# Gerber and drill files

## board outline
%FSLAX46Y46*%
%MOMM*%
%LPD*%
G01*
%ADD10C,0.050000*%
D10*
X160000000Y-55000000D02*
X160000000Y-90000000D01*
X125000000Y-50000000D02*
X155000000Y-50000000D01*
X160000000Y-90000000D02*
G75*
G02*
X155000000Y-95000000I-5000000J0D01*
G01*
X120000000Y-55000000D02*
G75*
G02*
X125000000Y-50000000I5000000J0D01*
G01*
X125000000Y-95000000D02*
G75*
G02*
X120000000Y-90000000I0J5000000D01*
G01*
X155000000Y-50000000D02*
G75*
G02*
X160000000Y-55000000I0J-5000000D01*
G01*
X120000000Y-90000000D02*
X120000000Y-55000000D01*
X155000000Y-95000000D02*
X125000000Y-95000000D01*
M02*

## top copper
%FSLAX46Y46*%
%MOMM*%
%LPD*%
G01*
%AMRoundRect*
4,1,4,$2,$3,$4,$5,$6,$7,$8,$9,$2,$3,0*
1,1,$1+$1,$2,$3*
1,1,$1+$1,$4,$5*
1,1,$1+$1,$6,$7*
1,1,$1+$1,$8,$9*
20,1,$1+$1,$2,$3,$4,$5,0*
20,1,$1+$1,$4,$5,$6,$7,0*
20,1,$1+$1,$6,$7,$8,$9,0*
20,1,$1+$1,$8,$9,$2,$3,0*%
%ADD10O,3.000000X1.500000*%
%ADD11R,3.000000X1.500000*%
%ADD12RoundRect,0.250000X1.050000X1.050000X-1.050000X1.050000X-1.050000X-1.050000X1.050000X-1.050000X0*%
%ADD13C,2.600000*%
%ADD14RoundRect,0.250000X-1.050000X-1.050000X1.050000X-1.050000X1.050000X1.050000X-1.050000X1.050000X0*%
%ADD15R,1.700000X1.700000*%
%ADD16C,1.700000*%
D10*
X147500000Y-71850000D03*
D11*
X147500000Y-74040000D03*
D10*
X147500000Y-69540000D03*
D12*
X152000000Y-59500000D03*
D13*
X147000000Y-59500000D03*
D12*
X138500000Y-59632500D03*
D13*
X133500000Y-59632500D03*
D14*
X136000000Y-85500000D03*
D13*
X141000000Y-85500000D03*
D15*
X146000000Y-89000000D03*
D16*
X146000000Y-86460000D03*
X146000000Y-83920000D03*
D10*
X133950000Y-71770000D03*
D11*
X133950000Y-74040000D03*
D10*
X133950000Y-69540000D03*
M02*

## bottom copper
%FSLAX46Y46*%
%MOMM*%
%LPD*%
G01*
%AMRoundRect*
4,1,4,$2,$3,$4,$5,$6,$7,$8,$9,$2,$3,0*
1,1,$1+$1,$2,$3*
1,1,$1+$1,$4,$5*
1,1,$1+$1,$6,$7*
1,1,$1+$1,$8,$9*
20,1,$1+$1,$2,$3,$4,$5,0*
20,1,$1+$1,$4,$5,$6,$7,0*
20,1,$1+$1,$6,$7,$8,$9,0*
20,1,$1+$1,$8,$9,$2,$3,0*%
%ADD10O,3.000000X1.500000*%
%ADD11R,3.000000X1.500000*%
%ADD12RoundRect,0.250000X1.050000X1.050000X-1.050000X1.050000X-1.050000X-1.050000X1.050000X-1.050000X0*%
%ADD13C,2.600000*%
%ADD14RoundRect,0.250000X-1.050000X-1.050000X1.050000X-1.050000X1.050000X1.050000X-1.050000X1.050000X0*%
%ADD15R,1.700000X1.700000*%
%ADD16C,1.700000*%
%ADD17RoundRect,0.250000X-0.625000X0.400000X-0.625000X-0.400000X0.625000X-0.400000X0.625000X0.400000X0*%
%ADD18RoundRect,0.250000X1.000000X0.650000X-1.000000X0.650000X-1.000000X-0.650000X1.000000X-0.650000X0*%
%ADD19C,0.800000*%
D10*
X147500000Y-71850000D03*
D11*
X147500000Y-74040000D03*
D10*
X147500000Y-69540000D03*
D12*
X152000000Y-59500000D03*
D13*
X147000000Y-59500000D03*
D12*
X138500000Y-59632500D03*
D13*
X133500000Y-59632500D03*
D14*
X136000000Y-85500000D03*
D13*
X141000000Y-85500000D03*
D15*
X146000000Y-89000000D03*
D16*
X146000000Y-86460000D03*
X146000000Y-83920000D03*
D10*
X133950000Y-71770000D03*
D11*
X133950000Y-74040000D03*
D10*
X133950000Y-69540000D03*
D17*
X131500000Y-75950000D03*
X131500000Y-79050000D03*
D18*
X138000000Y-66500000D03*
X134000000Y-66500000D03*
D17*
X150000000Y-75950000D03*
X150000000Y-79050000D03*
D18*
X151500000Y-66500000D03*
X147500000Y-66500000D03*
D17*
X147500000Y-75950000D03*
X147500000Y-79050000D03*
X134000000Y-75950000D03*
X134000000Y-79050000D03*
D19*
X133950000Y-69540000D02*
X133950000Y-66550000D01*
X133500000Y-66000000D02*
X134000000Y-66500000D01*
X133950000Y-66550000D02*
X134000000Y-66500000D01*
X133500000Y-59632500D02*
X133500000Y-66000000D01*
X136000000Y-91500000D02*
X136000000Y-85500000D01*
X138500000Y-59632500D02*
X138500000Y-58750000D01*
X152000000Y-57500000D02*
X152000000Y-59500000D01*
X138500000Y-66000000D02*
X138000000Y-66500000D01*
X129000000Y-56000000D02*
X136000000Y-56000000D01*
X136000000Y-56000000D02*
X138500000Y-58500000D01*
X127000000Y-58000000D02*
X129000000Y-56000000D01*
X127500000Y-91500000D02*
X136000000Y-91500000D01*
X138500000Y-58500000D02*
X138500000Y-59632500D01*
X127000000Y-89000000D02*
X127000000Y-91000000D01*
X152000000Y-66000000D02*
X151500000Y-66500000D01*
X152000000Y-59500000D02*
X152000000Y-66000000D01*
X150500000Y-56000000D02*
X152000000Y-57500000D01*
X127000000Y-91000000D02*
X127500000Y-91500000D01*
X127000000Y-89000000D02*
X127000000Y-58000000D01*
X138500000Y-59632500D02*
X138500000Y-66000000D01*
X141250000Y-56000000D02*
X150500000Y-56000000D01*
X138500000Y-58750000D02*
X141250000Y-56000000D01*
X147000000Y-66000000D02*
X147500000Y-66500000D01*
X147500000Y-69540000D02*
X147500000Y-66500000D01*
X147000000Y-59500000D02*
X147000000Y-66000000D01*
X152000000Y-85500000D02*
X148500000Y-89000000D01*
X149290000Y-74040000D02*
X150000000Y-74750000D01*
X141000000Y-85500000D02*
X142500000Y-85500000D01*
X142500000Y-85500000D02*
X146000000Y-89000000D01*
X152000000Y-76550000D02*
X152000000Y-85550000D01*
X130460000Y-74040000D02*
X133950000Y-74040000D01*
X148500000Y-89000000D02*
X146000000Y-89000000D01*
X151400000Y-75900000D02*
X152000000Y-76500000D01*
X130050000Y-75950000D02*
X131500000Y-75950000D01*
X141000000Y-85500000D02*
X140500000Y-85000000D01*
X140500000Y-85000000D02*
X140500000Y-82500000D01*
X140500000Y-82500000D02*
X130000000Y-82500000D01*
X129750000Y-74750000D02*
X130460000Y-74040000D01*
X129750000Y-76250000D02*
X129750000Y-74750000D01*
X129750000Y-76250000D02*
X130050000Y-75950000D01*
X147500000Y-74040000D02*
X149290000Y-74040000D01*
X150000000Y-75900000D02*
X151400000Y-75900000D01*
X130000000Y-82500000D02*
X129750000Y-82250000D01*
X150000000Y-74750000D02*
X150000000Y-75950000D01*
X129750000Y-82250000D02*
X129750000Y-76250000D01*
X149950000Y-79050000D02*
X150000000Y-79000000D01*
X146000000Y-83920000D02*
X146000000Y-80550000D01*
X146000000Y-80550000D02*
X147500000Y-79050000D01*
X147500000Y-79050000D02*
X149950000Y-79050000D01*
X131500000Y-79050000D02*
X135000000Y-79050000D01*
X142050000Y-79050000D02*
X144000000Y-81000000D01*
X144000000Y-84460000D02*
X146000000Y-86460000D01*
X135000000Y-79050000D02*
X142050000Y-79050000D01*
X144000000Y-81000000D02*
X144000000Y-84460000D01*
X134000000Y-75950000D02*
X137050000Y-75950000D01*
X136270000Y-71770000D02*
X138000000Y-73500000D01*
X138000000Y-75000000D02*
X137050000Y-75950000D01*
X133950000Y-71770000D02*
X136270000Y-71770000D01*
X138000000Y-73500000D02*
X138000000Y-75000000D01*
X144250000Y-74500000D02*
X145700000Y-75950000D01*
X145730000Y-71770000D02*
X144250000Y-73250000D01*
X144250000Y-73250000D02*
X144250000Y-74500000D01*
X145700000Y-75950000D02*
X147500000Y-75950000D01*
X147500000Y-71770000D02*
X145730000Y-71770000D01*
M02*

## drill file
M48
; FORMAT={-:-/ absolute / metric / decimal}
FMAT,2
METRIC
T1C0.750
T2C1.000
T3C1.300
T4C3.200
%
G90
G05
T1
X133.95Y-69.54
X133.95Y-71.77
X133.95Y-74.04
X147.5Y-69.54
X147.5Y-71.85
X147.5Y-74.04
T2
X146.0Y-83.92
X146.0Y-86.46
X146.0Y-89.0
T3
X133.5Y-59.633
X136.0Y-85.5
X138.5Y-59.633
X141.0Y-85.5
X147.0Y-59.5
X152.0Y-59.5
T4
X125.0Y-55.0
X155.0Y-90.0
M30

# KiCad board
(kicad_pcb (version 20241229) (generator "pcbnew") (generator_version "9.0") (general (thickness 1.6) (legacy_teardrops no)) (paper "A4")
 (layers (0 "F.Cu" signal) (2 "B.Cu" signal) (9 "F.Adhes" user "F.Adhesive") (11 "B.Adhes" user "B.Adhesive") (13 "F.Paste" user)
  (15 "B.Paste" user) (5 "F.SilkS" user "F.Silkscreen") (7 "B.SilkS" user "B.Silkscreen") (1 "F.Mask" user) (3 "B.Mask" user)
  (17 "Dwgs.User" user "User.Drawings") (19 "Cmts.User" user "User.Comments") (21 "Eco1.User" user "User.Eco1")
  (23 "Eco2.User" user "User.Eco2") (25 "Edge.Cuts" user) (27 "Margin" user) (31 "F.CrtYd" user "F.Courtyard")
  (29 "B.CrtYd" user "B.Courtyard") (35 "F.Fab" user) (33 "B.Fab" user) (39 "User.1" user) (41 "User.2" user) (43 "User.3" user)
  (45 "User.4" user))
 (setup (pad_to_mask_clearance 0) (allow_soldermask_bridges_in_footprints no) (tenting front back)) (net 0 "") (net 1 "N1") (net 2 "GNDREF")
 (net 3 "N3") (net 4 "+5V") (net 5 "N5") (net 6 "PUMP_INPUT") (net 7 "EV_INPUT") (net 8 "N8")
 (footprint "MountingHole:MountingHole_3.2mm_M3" (layer "F.Cu") (at 125 55 180)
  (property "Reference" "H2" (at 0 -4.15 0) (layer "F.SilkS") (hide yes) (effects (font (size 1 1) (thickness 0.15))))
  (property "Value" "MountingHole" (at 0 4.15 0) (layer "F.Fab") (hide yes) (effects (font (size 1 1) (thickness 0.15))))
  (pad "" np_thru_hole circle (at 0 0 180) (size 3.2 3.2) (drill 3.2) (layers "*.Cu" "*.Mask")))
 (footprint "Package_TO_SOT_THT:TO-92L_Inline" (layer "F.Cu") (at 147.5 73.04 90)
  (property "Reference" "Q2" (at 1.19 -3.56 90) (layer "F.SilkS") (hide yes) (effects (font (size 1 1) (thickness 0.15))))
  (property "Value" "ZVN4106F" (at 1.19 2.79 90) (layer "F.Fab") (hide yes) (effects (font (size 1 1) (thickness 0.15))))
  (pad "1" thru_hole oval (at 1.19 0 90) (size 1.5 3) (drill 0.75) (layers "*.Cu" "*.Mask") (remove_unused_layers no) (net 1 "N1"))
  (pad "2" thru_hole rect (at -1 0 90) (size 1.5 3) (drill 0.75) (layers "*.Cu" "*.Mask") (remove_unused_layers no) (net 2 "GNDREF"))
  (pad "3" thru_hole oval (at 3.5 0 90) (size 1.5 3) (drill 0.75) (layers "*.Cu" "*.Mask") (remove_unused_layers no) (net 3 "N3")))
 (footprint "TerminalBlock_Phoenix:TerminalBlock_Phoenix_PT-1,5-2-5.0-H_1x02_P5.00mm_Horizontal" (layer "F.Cu") (at 152 59.5 180)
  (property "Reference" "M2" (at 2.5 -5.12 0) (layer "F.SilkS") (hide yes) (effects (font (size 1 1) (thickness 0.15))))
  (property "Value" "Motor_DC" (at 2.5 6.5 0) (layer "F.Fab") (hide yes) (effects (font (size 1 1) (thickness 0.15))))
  (pad "1" thru_hole roundrect (at 0 0 180) (size 2.6 2.6) (drill 1.3) (layers "*.Cu" "*.Mask") (remove_unused_layers no)
   (roundrect_rratio 0.096154) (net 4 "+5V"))
  (pad "2" thru_hole circle (at 5 0 180) (size 2.6 2.6) (drill 1.3) (layers "*.Cu" "*.Mask") (remove_unused_layers no) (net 3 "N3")))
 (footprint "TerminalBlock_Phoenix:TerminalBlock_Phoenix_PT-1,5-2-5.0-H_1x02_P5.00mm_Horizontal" (layer "F.Cu") (at 138.5 59.6325 180)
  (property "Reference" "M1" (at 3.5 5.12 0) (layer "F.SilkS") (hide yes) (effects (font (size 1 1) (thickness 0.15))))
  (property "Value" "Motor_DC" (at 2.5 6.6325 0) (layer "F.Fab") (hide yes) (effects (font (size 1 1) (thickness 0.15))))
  (pad "1" thru_hole roundrect (at 0 0 180) (size 2.6 2.6) (drill 1.3) (layers "*.Cu" "*.Mask") (remove_unused_layers no)
   (roundrect_rratio 0.096154) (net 4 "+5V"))
  (pad "2" thru_hole circle (at 5 0 180) (size 2.6 2.6) (drill 1.3) (layers "*.Cu" "*.Mask") (remove_unused_layers no) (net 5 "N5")))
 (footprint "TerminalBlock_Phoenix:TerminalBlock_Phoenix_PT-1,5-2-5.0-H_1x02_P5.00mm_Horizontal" (layer "F.Cu") (at 136 85.5)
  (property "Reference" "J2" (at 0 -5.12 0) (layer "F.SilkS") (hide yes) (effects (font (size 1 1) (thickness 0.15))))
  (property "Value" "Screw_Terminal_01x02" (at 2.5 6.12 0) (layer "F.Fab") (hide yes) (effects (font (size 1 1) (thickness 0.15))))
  (pad "1" thru_hole roundrect (at 0 0) (size 2.6 2.6) (drill 1.3) (layers "*.Cu" "*.Mask") (remove_unused_layers no)
   (roundrect_rratio 0.096154) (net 4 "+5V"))
  (pad "2" thru_hole circle (at 5 0) (size 2.6 2.6) (drill 1.3) (layers "*.Cu" "*.Mask") (remove_unused_layers no) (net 2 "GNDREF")))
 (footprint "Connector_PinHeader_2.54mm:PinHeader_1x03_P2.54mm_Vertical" (layer "F.Cu") (at 146 89 180)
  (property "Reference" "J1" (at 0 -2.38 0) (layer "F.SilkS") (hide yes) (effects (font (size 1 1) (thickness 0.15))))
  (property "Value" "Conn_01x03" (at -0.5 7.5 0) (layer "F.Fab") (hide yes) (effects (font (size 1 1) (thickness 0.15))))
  (pad "1" thru_hole rect (at 0 0 180) (size 1.7 1.7) (drill 1) (layers "*.Cu" "*.Mask") (remove_unused_layers no) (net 2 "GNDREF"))
  (pad "2" thru_hole circle (at 0 2.54 180) (size 1.7 1.7) (drill 1) (layers "*.Cu" "*.Mask") (remove_unused_layers no) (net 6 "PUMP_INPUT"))
  (pad "3" thru_hole circle (at 0 5.08 180) (size 1.7 1.7) (drill 1) (layers "*.Cu" "*.Mask") (remove_unused_layers no) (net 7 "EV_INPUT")))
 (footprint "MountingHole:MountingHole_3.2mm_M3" (layer "F.Cu") (at 155 90 90)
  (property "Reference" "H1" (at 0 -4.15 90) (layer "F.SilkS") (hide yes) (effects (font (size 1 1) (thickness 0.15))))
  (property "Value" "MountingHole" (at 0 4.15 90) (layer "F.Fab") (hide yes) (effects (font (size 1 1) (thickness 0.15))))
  (pad "" np_thru_hole circle (at 0 0 90) (size 3.2 3.2) (drill 3.2) (layers "*.Cu" "*.Mask")))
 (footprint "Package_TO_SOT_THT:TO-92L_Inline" (layer "F.Cu") (at 133.95 73.04 90)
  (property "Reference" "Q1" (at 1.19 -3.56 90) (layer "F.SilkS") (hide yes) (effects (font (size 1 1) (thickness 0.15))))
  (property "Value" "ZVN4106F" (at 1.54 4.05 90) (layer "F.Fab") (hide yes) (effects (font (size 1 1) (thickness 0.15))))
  (pad "1" thru_hole oval (at 1.27 0 90) (size 1.5 3) (drill 0.75) (layers "*.Cu" "*.Mask") (remove_unused_layers no) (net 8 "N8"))
  (pad "2" thru_hole rect (at -1 0 90) (size 1.5 3) (drill 0.75) (layers "*.Cu" "*.Mask") (remove_unused_layers no) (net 2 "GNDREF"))
  (pad "3" thru_hole oval (at 3.5 0 90) (size 1.5 3) (drill 0.75) (layers "*.Cu" "*.Mask") (remove_unused_layers no) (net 5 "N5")))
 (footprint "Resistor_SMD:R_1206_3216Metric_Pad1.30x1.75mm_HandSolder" (layer "B.Cu") (at 131.5 77.5 -90)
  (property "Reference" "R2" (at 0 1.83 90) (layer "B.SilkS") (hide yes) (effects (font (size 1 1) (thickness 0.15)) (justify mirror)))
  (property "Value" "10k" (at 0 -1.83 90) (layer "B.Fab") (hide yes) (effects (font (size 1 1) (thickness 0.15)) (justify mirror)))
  (pad "1" smd roundrect (at -1.55 0 270) (size 1.3 1.75) (layers "B.Cu" "B.Mask" "B.Paste") (roundrect_rratio 0.192308) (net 2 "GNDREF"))
  (pad "2" smd roundrect (at 1.55 0 270) (size 1.3 1.75) (layers "B.Cu" "B.Mask" "B.Paste") (roundrect_rratio 0.192308) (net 6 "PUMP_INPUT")))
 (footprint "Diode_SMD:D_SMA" (layer "B.Cu") (at 136 66.5 180)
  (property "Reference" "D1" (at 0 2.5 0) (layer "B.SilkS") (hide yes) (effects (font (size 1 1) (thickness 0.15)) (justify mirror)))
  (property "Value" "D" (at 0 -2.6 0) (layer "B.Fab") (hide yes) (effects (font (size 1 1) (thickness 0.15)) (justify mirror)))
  (pad "1" smd roundrect (at -2 0 180) (size 2.5 1.8) (layers "B.Cu" "B.Mask" "B.Paste") (roundrect_rratio 0.1388888889) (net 4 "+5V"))
  (pad "2" smd roundrect (at 2 0 180) (size 2.5 1.8) (layers "B.Cu" "B.Mask" "B.Paste") (roundrect_rratio 0.1388888889) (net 5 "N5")))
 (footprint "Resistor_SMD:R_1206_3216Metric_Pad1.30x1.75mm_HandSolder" (layer "B.Cu") (at 150 77.5 -90)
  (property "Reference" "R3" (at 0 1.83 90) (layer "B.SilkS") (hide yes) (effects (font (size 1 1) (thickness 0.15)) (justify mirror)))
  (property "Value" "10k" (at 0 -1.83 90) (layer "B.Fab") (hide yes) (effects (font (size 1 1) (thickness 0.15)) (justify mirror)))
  (pad "1" smd roundrect (at -1.55 0 270) (size 1.3 1.75) (layers "B.Cu" "B.Mask" "B.Paste") (roundrect_rratio 0.192308) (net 2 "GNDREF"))
  (pad "2" smd roundrect (at 1.55 0 270) (size 1.3 1.75) (layers "B.Cu" "B.Mask" "B.Paste") (roundrect_rratio 0.192308) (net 7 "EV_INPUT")))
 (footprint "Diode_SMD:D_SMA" (layer "B.Cu") (at 149.5 66.5 180)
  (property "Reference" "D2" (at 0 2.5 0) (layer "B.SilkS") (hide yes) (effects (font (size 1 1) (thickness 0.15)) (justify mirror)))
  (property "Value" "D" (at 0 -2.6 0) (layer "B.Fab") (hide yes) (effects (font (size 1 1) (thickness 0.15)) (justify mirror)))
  (pad "1" smd roundrect (at -2 0 180) (size 2.5 1.8) (layers "B.Cu" "B.Mask" "B.Paste") (roundrect_rratio 0.1388888889) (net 4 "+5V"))
  (pad "2" smd roundrect (at 2 0 180) (size 2.5 1.8) (layers "B.Cu" "B.Mask" "B.Paste") (roundrect_rratio 0.1388888889) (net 3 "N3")))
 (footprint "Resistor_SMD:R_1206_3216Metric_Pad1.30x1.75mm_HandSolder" (layer "B.Cu") (at 147.5 77.5 -90)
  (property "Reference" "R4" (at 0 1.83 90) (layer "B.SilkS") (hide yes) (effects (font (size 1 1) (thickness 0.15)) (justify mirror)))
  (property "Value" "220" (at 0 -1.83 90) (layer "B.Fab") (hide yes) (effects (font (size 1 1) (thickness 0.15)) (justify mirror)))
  (pad "1" smd roundrect (at -1.55 0 270) (size 1.3 1.75) (layers "B.Cu" "B.Mask" "B.Paste") (roundrect_rratio 0.192308) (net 1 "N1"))
  (pad "2" smd roundrect (at 1.55 0 270) (size 1.3 1.75) (layers "B.Cu" "B.Mask" "B.Paste") (roundrect_rratio 0.192308) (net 7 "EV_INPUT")))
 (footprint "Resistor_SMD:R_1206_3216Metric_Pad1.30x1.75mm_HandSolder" (layer "B.Cu") (at 134 77.5 -90)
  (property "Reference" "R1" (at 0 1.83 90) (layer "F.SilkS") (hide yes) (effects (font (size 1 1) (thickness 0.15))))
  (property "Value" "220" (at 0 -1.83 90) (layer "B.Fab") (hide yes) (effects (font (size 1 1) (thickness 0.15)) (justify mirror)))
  (pad "1" smd roundrect (at -1.55 0 270) (size 1.3 1.75) (layers "B.Cu" "B.Mask" "B.Paste") (roundrect_rratio 0.192308) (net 8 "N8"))
  (pad "2" smd roundrect (at 1.55 0 270) (size 1.3 1.75) (layers "B.Cu" "B.Mask" "B.Paste") (roundrect_rratio 0.192308) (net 6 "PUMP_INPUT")))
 (gr_line (start 160 55) (end 160 90) (stroke (width 0.05) (type default)) (layer "Edge.Cuts"))
 (gr_line (start 125 50) (end 155 50) (stroke (width 0.05) (type default)) (layer "Edge.Cuts"))
 (gr_arc (start 160 90) (mid 158.535534 93.535534) (end 155 95) (stroke (width 0.05) (type default)) (layer "Edge.Cuts"))
 (gr_arc (start 120 55) (mid 121.464466 51.464466) (end 125 50) (stroke (width 0.05) (type default)) (layer "Edge.Cuts"))
 (gr_arc (start 125 95) (mid 121.464466 93.535534) (end 120 90) (stroke (width 0.05) (type default)) (layer "Edge.Cuts"))
 (gr_arc (start 155 50) (mid 158.535534 51.464466) (end 160 55) (stroke (width 0.05) (type default)) (layer "Edge.Cuts"))
 (gr_line (start 120 90) (end 120 55) (stroke (width 0.05) (type default)) (layer "Edge.Cuts"))
 (gr_line (start 155 95) (end 125 95) (stroke (width 0.05) (type default)) (layer "Edge.Cuts"))
 (segment (start 133.95 69.54) (end 133.95 66.55) (width 0.8) (layer "B.Cu") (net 5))
 (segment (start 133.5 66) (end 134 66.5) (width 0.8) (layer "B.Cu") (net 5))
 (segment (start 133.95 66.55) (end 134 66.5) (width 0.8) (layer "B.Cu") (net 5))
 (segment (start 133.5 59.6325) (end 133.5 66) (width 0.8) (layer "B.Cu") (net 5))
 (segment (start 136 91.5) (end 136 85.5) (width 0.8) (layer "B.Cu") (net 4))
 (segment (start 138.5 59.6325) (end 138.5 58.75) (width 0.8) (layer "B.Cu") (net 4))
 (segment (start 152 57.5) (end 152 59.5) (width 0.8) (layer "B.Cu") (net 4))
 (segment (start 138.5 66) (end 138 66.5) (width 0.8) (layer "B.Cu") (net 4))
 (segment (start 129 56) (end 136 56) (width 0.8) (layer "B.Cu") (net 4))
 (segment (start 136 56) (end 138.5 58.5) (width 0.8) (layer "B.Cu") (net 4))
 (segment (start 127 58) (end 129 56) (width 0.8) (layer "B.Cu") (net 4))
 (segment (start 127.5 91.5) (end 136 91.5) (width 0.8) (layer "B.Cu") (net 4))
 (segment (start 138.5 58.5) (end 138.5 59.6325) (width 0.8) (layer "B.Cu") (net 4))
 (segment (start 127 89) (end 127 91) (width 0.8) (layer "B.Cu") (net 4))
 (segment (start 152 66) (end 151.5 66.5) (width 0.8) (layer "B.Cu") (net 4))
 (segment (start 152 59.5) (end 152 66) (width 0.8) (layer "B.Cu") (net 4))
 (segment (start 150.5 56) (end 152 57.5) (width 0.8) (layer "B.Cu") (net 4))
 (segment (start 127 91) (end 127.5 91.5) (width 0.8) (layer "B.Cu") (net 4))
 (segment (start 127 89) (end 127 58) (width 0.8) (layer "B.Cu") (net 4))
 (segment (start 138.5 59.6325) (end 138.5 66) (width 0.8) (layer "B.Cu") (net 4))
 (segment (start 141.25 56) (end 150.5 56) (width 0.8) (layer "B.Cu") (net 4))
 (segment (start 138.5 58.75) (end 141.25 56) (width 0.8) (layer "B.Cu") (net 4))
 (segment (start 147 66) (end 147.5 66.5) (width 0.8) (layer "B.Cu") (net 3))
 (segment (start 147.5 69.54) (end 147.5 66.5) (width 0.8) (layer "B.Cu") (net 3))
 (segment (start 147 59.5) (end 147 66) (width 0.8) (layer "B.Cu") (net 3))
 (segment (start 152 85.5) (end 148.5 89) (width 0.8) (layer "B.Cu") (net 2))
 (segment (start 149.29 74.04) (end 150 74.75) (width 0.8) (layer "B.Cu") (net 2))
 (segment (start 141 85.5) (end 142.5 85.5) (width 0.8) (layer "B.Cu") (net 2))
 (segment (start 142.5 85.5) (end 146 89) (width 0.8) (layer "B.Cu") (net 2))
 (segment (start 152 76.55) (end 152 85.55) (width 0.8) (layer "B.Cu") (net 2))
 (segment (start 130.46 74.04) (end 133.95 74.04) (width 0.8) (layer "B.Cu") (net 2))
 (segment (start 148.5 89) (end 146 89) (width 0.8) (layer "B.Cu") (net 2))
 (segment (start 151.4 75.9) (end 152 76.5) (width 0.8) (layer "B.Cu") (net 2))
 (segment (start 130.05 75.95) (end 131.5 75.95) (width 0.8) (layer "B.Cu") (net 2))
 (segment (start 141 85.5) (end 140.5 85) (width 0.8) (layer "B.Cu") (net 2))
 (segment (start 140.5 85) (end 140.5 82.5) (width 0.8) (layer "B.Cu") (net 2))
 (segment (start 140.5 82.5) (end 130 82.5) (width 0.8) (layer "B.Cu") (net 2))
 (segment (start 129.75 74.75) (end 130.46 74.04) (width 0.8) (layer "B.Cu") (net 2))
 (segment (start 129.75 76.25) (end 129.75 74.75) (width 0.8) (layer "B.Cu") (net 2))
 (segment (start 129.75 76.25) (end 130.05 75.95) (width 0.8) (layer "B.Cu") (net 2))
 (segment (start 147.5 74.04) (end 149.29 74.04) (width 0.8) (layer "B.Cu") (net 2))
 (segment (start 150 75.9) (end 151.4 75.9) (width 0.8) (layer "B.Cu") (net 2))
 (segment (start 130 82.5) (end 129.75 82.25) (width 0.8) (layer "B.Cu") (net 2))
 (segment (start 150 74.75) (end 150 75.95) (width 0.8) (layer "B.Cu") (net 2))
 (segment (start 129.75 82.25) (end 129.75 76.25) (width 0.8) (layer "B.Cu") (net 2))
 (segment (start 149.95 79.05) (end 150 79) (width 0.8) (layer "B.Cu") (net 7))
 (segment (start 146 83.92) (end 146 80.55) (width 0.8) (layer "B.Cu") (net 7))
 (segment (start 146 80.55) (end 147.5 79.05) (width 0.8) (layer "B.Cu") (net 7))
 (segment (start 147.5 79.05) (end 149.95 79.05) (width 0.8) (layer "B.Cu") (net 7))
 (segment (start 131.5 79.05) (end 135 79.05) (width 0.8) (layer "B.Cu") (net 6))
 (segment (start 142.05 79.05) (end 144 81) (width 0.8) (layer "B.Cu") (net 6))
 (segment (start 144 84.46) (end 146 86.46) (width 0.8) (layer "B.Cu") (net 6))
 (segment (start 135 79.05) (end 142.05 79.05) (width 0.8) (layer "B.Cu") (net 6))
 (segment (start 144 81) (end 144 84.46) (width 0.8) (layer "B.Cu") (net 6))
 (segment (start 134 75.95) (end 137.05 75.95) (width 0.8) (layer "B.Cu") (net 8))
 (segment (start 136.27 71.77) (end 138 73.5) (width 0.8) (layer "B.Cu") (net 8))
 (segment (start 138 75) (end 137.05 75.95) (width 0.8) (layer "B.Cu") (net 8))
 (segment (start 133.95 71.77) (end 136.27 71.77) (width 0.8) (layer "B.Cu") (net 8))
 (segment (start 138 73.5) (end 138 75) (width 0.8) (layer "B.Cu") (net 8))
 (segment (start 144.25 74.5) (end 145.7 75.95) (width 0.8) (layer "B.Cu") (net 1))
 (segment (start 145.73 71.77) (end 144.25 73.25) (width 0.8) (layer "B.Cu") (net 1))
 (segment (start 144.25 73.25) (end 144.25 74.5) (width 0.8) (layer "B.Cu") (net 1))
 (segment (start 145.7 75.95) (end 147.5 75.95) (width 0.8) (layer "B.Cu") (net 1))
 (segment (start 147.5 71.77) (end 145.73 71.77) (width 0.8) (layer "B.Cu") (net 1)))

